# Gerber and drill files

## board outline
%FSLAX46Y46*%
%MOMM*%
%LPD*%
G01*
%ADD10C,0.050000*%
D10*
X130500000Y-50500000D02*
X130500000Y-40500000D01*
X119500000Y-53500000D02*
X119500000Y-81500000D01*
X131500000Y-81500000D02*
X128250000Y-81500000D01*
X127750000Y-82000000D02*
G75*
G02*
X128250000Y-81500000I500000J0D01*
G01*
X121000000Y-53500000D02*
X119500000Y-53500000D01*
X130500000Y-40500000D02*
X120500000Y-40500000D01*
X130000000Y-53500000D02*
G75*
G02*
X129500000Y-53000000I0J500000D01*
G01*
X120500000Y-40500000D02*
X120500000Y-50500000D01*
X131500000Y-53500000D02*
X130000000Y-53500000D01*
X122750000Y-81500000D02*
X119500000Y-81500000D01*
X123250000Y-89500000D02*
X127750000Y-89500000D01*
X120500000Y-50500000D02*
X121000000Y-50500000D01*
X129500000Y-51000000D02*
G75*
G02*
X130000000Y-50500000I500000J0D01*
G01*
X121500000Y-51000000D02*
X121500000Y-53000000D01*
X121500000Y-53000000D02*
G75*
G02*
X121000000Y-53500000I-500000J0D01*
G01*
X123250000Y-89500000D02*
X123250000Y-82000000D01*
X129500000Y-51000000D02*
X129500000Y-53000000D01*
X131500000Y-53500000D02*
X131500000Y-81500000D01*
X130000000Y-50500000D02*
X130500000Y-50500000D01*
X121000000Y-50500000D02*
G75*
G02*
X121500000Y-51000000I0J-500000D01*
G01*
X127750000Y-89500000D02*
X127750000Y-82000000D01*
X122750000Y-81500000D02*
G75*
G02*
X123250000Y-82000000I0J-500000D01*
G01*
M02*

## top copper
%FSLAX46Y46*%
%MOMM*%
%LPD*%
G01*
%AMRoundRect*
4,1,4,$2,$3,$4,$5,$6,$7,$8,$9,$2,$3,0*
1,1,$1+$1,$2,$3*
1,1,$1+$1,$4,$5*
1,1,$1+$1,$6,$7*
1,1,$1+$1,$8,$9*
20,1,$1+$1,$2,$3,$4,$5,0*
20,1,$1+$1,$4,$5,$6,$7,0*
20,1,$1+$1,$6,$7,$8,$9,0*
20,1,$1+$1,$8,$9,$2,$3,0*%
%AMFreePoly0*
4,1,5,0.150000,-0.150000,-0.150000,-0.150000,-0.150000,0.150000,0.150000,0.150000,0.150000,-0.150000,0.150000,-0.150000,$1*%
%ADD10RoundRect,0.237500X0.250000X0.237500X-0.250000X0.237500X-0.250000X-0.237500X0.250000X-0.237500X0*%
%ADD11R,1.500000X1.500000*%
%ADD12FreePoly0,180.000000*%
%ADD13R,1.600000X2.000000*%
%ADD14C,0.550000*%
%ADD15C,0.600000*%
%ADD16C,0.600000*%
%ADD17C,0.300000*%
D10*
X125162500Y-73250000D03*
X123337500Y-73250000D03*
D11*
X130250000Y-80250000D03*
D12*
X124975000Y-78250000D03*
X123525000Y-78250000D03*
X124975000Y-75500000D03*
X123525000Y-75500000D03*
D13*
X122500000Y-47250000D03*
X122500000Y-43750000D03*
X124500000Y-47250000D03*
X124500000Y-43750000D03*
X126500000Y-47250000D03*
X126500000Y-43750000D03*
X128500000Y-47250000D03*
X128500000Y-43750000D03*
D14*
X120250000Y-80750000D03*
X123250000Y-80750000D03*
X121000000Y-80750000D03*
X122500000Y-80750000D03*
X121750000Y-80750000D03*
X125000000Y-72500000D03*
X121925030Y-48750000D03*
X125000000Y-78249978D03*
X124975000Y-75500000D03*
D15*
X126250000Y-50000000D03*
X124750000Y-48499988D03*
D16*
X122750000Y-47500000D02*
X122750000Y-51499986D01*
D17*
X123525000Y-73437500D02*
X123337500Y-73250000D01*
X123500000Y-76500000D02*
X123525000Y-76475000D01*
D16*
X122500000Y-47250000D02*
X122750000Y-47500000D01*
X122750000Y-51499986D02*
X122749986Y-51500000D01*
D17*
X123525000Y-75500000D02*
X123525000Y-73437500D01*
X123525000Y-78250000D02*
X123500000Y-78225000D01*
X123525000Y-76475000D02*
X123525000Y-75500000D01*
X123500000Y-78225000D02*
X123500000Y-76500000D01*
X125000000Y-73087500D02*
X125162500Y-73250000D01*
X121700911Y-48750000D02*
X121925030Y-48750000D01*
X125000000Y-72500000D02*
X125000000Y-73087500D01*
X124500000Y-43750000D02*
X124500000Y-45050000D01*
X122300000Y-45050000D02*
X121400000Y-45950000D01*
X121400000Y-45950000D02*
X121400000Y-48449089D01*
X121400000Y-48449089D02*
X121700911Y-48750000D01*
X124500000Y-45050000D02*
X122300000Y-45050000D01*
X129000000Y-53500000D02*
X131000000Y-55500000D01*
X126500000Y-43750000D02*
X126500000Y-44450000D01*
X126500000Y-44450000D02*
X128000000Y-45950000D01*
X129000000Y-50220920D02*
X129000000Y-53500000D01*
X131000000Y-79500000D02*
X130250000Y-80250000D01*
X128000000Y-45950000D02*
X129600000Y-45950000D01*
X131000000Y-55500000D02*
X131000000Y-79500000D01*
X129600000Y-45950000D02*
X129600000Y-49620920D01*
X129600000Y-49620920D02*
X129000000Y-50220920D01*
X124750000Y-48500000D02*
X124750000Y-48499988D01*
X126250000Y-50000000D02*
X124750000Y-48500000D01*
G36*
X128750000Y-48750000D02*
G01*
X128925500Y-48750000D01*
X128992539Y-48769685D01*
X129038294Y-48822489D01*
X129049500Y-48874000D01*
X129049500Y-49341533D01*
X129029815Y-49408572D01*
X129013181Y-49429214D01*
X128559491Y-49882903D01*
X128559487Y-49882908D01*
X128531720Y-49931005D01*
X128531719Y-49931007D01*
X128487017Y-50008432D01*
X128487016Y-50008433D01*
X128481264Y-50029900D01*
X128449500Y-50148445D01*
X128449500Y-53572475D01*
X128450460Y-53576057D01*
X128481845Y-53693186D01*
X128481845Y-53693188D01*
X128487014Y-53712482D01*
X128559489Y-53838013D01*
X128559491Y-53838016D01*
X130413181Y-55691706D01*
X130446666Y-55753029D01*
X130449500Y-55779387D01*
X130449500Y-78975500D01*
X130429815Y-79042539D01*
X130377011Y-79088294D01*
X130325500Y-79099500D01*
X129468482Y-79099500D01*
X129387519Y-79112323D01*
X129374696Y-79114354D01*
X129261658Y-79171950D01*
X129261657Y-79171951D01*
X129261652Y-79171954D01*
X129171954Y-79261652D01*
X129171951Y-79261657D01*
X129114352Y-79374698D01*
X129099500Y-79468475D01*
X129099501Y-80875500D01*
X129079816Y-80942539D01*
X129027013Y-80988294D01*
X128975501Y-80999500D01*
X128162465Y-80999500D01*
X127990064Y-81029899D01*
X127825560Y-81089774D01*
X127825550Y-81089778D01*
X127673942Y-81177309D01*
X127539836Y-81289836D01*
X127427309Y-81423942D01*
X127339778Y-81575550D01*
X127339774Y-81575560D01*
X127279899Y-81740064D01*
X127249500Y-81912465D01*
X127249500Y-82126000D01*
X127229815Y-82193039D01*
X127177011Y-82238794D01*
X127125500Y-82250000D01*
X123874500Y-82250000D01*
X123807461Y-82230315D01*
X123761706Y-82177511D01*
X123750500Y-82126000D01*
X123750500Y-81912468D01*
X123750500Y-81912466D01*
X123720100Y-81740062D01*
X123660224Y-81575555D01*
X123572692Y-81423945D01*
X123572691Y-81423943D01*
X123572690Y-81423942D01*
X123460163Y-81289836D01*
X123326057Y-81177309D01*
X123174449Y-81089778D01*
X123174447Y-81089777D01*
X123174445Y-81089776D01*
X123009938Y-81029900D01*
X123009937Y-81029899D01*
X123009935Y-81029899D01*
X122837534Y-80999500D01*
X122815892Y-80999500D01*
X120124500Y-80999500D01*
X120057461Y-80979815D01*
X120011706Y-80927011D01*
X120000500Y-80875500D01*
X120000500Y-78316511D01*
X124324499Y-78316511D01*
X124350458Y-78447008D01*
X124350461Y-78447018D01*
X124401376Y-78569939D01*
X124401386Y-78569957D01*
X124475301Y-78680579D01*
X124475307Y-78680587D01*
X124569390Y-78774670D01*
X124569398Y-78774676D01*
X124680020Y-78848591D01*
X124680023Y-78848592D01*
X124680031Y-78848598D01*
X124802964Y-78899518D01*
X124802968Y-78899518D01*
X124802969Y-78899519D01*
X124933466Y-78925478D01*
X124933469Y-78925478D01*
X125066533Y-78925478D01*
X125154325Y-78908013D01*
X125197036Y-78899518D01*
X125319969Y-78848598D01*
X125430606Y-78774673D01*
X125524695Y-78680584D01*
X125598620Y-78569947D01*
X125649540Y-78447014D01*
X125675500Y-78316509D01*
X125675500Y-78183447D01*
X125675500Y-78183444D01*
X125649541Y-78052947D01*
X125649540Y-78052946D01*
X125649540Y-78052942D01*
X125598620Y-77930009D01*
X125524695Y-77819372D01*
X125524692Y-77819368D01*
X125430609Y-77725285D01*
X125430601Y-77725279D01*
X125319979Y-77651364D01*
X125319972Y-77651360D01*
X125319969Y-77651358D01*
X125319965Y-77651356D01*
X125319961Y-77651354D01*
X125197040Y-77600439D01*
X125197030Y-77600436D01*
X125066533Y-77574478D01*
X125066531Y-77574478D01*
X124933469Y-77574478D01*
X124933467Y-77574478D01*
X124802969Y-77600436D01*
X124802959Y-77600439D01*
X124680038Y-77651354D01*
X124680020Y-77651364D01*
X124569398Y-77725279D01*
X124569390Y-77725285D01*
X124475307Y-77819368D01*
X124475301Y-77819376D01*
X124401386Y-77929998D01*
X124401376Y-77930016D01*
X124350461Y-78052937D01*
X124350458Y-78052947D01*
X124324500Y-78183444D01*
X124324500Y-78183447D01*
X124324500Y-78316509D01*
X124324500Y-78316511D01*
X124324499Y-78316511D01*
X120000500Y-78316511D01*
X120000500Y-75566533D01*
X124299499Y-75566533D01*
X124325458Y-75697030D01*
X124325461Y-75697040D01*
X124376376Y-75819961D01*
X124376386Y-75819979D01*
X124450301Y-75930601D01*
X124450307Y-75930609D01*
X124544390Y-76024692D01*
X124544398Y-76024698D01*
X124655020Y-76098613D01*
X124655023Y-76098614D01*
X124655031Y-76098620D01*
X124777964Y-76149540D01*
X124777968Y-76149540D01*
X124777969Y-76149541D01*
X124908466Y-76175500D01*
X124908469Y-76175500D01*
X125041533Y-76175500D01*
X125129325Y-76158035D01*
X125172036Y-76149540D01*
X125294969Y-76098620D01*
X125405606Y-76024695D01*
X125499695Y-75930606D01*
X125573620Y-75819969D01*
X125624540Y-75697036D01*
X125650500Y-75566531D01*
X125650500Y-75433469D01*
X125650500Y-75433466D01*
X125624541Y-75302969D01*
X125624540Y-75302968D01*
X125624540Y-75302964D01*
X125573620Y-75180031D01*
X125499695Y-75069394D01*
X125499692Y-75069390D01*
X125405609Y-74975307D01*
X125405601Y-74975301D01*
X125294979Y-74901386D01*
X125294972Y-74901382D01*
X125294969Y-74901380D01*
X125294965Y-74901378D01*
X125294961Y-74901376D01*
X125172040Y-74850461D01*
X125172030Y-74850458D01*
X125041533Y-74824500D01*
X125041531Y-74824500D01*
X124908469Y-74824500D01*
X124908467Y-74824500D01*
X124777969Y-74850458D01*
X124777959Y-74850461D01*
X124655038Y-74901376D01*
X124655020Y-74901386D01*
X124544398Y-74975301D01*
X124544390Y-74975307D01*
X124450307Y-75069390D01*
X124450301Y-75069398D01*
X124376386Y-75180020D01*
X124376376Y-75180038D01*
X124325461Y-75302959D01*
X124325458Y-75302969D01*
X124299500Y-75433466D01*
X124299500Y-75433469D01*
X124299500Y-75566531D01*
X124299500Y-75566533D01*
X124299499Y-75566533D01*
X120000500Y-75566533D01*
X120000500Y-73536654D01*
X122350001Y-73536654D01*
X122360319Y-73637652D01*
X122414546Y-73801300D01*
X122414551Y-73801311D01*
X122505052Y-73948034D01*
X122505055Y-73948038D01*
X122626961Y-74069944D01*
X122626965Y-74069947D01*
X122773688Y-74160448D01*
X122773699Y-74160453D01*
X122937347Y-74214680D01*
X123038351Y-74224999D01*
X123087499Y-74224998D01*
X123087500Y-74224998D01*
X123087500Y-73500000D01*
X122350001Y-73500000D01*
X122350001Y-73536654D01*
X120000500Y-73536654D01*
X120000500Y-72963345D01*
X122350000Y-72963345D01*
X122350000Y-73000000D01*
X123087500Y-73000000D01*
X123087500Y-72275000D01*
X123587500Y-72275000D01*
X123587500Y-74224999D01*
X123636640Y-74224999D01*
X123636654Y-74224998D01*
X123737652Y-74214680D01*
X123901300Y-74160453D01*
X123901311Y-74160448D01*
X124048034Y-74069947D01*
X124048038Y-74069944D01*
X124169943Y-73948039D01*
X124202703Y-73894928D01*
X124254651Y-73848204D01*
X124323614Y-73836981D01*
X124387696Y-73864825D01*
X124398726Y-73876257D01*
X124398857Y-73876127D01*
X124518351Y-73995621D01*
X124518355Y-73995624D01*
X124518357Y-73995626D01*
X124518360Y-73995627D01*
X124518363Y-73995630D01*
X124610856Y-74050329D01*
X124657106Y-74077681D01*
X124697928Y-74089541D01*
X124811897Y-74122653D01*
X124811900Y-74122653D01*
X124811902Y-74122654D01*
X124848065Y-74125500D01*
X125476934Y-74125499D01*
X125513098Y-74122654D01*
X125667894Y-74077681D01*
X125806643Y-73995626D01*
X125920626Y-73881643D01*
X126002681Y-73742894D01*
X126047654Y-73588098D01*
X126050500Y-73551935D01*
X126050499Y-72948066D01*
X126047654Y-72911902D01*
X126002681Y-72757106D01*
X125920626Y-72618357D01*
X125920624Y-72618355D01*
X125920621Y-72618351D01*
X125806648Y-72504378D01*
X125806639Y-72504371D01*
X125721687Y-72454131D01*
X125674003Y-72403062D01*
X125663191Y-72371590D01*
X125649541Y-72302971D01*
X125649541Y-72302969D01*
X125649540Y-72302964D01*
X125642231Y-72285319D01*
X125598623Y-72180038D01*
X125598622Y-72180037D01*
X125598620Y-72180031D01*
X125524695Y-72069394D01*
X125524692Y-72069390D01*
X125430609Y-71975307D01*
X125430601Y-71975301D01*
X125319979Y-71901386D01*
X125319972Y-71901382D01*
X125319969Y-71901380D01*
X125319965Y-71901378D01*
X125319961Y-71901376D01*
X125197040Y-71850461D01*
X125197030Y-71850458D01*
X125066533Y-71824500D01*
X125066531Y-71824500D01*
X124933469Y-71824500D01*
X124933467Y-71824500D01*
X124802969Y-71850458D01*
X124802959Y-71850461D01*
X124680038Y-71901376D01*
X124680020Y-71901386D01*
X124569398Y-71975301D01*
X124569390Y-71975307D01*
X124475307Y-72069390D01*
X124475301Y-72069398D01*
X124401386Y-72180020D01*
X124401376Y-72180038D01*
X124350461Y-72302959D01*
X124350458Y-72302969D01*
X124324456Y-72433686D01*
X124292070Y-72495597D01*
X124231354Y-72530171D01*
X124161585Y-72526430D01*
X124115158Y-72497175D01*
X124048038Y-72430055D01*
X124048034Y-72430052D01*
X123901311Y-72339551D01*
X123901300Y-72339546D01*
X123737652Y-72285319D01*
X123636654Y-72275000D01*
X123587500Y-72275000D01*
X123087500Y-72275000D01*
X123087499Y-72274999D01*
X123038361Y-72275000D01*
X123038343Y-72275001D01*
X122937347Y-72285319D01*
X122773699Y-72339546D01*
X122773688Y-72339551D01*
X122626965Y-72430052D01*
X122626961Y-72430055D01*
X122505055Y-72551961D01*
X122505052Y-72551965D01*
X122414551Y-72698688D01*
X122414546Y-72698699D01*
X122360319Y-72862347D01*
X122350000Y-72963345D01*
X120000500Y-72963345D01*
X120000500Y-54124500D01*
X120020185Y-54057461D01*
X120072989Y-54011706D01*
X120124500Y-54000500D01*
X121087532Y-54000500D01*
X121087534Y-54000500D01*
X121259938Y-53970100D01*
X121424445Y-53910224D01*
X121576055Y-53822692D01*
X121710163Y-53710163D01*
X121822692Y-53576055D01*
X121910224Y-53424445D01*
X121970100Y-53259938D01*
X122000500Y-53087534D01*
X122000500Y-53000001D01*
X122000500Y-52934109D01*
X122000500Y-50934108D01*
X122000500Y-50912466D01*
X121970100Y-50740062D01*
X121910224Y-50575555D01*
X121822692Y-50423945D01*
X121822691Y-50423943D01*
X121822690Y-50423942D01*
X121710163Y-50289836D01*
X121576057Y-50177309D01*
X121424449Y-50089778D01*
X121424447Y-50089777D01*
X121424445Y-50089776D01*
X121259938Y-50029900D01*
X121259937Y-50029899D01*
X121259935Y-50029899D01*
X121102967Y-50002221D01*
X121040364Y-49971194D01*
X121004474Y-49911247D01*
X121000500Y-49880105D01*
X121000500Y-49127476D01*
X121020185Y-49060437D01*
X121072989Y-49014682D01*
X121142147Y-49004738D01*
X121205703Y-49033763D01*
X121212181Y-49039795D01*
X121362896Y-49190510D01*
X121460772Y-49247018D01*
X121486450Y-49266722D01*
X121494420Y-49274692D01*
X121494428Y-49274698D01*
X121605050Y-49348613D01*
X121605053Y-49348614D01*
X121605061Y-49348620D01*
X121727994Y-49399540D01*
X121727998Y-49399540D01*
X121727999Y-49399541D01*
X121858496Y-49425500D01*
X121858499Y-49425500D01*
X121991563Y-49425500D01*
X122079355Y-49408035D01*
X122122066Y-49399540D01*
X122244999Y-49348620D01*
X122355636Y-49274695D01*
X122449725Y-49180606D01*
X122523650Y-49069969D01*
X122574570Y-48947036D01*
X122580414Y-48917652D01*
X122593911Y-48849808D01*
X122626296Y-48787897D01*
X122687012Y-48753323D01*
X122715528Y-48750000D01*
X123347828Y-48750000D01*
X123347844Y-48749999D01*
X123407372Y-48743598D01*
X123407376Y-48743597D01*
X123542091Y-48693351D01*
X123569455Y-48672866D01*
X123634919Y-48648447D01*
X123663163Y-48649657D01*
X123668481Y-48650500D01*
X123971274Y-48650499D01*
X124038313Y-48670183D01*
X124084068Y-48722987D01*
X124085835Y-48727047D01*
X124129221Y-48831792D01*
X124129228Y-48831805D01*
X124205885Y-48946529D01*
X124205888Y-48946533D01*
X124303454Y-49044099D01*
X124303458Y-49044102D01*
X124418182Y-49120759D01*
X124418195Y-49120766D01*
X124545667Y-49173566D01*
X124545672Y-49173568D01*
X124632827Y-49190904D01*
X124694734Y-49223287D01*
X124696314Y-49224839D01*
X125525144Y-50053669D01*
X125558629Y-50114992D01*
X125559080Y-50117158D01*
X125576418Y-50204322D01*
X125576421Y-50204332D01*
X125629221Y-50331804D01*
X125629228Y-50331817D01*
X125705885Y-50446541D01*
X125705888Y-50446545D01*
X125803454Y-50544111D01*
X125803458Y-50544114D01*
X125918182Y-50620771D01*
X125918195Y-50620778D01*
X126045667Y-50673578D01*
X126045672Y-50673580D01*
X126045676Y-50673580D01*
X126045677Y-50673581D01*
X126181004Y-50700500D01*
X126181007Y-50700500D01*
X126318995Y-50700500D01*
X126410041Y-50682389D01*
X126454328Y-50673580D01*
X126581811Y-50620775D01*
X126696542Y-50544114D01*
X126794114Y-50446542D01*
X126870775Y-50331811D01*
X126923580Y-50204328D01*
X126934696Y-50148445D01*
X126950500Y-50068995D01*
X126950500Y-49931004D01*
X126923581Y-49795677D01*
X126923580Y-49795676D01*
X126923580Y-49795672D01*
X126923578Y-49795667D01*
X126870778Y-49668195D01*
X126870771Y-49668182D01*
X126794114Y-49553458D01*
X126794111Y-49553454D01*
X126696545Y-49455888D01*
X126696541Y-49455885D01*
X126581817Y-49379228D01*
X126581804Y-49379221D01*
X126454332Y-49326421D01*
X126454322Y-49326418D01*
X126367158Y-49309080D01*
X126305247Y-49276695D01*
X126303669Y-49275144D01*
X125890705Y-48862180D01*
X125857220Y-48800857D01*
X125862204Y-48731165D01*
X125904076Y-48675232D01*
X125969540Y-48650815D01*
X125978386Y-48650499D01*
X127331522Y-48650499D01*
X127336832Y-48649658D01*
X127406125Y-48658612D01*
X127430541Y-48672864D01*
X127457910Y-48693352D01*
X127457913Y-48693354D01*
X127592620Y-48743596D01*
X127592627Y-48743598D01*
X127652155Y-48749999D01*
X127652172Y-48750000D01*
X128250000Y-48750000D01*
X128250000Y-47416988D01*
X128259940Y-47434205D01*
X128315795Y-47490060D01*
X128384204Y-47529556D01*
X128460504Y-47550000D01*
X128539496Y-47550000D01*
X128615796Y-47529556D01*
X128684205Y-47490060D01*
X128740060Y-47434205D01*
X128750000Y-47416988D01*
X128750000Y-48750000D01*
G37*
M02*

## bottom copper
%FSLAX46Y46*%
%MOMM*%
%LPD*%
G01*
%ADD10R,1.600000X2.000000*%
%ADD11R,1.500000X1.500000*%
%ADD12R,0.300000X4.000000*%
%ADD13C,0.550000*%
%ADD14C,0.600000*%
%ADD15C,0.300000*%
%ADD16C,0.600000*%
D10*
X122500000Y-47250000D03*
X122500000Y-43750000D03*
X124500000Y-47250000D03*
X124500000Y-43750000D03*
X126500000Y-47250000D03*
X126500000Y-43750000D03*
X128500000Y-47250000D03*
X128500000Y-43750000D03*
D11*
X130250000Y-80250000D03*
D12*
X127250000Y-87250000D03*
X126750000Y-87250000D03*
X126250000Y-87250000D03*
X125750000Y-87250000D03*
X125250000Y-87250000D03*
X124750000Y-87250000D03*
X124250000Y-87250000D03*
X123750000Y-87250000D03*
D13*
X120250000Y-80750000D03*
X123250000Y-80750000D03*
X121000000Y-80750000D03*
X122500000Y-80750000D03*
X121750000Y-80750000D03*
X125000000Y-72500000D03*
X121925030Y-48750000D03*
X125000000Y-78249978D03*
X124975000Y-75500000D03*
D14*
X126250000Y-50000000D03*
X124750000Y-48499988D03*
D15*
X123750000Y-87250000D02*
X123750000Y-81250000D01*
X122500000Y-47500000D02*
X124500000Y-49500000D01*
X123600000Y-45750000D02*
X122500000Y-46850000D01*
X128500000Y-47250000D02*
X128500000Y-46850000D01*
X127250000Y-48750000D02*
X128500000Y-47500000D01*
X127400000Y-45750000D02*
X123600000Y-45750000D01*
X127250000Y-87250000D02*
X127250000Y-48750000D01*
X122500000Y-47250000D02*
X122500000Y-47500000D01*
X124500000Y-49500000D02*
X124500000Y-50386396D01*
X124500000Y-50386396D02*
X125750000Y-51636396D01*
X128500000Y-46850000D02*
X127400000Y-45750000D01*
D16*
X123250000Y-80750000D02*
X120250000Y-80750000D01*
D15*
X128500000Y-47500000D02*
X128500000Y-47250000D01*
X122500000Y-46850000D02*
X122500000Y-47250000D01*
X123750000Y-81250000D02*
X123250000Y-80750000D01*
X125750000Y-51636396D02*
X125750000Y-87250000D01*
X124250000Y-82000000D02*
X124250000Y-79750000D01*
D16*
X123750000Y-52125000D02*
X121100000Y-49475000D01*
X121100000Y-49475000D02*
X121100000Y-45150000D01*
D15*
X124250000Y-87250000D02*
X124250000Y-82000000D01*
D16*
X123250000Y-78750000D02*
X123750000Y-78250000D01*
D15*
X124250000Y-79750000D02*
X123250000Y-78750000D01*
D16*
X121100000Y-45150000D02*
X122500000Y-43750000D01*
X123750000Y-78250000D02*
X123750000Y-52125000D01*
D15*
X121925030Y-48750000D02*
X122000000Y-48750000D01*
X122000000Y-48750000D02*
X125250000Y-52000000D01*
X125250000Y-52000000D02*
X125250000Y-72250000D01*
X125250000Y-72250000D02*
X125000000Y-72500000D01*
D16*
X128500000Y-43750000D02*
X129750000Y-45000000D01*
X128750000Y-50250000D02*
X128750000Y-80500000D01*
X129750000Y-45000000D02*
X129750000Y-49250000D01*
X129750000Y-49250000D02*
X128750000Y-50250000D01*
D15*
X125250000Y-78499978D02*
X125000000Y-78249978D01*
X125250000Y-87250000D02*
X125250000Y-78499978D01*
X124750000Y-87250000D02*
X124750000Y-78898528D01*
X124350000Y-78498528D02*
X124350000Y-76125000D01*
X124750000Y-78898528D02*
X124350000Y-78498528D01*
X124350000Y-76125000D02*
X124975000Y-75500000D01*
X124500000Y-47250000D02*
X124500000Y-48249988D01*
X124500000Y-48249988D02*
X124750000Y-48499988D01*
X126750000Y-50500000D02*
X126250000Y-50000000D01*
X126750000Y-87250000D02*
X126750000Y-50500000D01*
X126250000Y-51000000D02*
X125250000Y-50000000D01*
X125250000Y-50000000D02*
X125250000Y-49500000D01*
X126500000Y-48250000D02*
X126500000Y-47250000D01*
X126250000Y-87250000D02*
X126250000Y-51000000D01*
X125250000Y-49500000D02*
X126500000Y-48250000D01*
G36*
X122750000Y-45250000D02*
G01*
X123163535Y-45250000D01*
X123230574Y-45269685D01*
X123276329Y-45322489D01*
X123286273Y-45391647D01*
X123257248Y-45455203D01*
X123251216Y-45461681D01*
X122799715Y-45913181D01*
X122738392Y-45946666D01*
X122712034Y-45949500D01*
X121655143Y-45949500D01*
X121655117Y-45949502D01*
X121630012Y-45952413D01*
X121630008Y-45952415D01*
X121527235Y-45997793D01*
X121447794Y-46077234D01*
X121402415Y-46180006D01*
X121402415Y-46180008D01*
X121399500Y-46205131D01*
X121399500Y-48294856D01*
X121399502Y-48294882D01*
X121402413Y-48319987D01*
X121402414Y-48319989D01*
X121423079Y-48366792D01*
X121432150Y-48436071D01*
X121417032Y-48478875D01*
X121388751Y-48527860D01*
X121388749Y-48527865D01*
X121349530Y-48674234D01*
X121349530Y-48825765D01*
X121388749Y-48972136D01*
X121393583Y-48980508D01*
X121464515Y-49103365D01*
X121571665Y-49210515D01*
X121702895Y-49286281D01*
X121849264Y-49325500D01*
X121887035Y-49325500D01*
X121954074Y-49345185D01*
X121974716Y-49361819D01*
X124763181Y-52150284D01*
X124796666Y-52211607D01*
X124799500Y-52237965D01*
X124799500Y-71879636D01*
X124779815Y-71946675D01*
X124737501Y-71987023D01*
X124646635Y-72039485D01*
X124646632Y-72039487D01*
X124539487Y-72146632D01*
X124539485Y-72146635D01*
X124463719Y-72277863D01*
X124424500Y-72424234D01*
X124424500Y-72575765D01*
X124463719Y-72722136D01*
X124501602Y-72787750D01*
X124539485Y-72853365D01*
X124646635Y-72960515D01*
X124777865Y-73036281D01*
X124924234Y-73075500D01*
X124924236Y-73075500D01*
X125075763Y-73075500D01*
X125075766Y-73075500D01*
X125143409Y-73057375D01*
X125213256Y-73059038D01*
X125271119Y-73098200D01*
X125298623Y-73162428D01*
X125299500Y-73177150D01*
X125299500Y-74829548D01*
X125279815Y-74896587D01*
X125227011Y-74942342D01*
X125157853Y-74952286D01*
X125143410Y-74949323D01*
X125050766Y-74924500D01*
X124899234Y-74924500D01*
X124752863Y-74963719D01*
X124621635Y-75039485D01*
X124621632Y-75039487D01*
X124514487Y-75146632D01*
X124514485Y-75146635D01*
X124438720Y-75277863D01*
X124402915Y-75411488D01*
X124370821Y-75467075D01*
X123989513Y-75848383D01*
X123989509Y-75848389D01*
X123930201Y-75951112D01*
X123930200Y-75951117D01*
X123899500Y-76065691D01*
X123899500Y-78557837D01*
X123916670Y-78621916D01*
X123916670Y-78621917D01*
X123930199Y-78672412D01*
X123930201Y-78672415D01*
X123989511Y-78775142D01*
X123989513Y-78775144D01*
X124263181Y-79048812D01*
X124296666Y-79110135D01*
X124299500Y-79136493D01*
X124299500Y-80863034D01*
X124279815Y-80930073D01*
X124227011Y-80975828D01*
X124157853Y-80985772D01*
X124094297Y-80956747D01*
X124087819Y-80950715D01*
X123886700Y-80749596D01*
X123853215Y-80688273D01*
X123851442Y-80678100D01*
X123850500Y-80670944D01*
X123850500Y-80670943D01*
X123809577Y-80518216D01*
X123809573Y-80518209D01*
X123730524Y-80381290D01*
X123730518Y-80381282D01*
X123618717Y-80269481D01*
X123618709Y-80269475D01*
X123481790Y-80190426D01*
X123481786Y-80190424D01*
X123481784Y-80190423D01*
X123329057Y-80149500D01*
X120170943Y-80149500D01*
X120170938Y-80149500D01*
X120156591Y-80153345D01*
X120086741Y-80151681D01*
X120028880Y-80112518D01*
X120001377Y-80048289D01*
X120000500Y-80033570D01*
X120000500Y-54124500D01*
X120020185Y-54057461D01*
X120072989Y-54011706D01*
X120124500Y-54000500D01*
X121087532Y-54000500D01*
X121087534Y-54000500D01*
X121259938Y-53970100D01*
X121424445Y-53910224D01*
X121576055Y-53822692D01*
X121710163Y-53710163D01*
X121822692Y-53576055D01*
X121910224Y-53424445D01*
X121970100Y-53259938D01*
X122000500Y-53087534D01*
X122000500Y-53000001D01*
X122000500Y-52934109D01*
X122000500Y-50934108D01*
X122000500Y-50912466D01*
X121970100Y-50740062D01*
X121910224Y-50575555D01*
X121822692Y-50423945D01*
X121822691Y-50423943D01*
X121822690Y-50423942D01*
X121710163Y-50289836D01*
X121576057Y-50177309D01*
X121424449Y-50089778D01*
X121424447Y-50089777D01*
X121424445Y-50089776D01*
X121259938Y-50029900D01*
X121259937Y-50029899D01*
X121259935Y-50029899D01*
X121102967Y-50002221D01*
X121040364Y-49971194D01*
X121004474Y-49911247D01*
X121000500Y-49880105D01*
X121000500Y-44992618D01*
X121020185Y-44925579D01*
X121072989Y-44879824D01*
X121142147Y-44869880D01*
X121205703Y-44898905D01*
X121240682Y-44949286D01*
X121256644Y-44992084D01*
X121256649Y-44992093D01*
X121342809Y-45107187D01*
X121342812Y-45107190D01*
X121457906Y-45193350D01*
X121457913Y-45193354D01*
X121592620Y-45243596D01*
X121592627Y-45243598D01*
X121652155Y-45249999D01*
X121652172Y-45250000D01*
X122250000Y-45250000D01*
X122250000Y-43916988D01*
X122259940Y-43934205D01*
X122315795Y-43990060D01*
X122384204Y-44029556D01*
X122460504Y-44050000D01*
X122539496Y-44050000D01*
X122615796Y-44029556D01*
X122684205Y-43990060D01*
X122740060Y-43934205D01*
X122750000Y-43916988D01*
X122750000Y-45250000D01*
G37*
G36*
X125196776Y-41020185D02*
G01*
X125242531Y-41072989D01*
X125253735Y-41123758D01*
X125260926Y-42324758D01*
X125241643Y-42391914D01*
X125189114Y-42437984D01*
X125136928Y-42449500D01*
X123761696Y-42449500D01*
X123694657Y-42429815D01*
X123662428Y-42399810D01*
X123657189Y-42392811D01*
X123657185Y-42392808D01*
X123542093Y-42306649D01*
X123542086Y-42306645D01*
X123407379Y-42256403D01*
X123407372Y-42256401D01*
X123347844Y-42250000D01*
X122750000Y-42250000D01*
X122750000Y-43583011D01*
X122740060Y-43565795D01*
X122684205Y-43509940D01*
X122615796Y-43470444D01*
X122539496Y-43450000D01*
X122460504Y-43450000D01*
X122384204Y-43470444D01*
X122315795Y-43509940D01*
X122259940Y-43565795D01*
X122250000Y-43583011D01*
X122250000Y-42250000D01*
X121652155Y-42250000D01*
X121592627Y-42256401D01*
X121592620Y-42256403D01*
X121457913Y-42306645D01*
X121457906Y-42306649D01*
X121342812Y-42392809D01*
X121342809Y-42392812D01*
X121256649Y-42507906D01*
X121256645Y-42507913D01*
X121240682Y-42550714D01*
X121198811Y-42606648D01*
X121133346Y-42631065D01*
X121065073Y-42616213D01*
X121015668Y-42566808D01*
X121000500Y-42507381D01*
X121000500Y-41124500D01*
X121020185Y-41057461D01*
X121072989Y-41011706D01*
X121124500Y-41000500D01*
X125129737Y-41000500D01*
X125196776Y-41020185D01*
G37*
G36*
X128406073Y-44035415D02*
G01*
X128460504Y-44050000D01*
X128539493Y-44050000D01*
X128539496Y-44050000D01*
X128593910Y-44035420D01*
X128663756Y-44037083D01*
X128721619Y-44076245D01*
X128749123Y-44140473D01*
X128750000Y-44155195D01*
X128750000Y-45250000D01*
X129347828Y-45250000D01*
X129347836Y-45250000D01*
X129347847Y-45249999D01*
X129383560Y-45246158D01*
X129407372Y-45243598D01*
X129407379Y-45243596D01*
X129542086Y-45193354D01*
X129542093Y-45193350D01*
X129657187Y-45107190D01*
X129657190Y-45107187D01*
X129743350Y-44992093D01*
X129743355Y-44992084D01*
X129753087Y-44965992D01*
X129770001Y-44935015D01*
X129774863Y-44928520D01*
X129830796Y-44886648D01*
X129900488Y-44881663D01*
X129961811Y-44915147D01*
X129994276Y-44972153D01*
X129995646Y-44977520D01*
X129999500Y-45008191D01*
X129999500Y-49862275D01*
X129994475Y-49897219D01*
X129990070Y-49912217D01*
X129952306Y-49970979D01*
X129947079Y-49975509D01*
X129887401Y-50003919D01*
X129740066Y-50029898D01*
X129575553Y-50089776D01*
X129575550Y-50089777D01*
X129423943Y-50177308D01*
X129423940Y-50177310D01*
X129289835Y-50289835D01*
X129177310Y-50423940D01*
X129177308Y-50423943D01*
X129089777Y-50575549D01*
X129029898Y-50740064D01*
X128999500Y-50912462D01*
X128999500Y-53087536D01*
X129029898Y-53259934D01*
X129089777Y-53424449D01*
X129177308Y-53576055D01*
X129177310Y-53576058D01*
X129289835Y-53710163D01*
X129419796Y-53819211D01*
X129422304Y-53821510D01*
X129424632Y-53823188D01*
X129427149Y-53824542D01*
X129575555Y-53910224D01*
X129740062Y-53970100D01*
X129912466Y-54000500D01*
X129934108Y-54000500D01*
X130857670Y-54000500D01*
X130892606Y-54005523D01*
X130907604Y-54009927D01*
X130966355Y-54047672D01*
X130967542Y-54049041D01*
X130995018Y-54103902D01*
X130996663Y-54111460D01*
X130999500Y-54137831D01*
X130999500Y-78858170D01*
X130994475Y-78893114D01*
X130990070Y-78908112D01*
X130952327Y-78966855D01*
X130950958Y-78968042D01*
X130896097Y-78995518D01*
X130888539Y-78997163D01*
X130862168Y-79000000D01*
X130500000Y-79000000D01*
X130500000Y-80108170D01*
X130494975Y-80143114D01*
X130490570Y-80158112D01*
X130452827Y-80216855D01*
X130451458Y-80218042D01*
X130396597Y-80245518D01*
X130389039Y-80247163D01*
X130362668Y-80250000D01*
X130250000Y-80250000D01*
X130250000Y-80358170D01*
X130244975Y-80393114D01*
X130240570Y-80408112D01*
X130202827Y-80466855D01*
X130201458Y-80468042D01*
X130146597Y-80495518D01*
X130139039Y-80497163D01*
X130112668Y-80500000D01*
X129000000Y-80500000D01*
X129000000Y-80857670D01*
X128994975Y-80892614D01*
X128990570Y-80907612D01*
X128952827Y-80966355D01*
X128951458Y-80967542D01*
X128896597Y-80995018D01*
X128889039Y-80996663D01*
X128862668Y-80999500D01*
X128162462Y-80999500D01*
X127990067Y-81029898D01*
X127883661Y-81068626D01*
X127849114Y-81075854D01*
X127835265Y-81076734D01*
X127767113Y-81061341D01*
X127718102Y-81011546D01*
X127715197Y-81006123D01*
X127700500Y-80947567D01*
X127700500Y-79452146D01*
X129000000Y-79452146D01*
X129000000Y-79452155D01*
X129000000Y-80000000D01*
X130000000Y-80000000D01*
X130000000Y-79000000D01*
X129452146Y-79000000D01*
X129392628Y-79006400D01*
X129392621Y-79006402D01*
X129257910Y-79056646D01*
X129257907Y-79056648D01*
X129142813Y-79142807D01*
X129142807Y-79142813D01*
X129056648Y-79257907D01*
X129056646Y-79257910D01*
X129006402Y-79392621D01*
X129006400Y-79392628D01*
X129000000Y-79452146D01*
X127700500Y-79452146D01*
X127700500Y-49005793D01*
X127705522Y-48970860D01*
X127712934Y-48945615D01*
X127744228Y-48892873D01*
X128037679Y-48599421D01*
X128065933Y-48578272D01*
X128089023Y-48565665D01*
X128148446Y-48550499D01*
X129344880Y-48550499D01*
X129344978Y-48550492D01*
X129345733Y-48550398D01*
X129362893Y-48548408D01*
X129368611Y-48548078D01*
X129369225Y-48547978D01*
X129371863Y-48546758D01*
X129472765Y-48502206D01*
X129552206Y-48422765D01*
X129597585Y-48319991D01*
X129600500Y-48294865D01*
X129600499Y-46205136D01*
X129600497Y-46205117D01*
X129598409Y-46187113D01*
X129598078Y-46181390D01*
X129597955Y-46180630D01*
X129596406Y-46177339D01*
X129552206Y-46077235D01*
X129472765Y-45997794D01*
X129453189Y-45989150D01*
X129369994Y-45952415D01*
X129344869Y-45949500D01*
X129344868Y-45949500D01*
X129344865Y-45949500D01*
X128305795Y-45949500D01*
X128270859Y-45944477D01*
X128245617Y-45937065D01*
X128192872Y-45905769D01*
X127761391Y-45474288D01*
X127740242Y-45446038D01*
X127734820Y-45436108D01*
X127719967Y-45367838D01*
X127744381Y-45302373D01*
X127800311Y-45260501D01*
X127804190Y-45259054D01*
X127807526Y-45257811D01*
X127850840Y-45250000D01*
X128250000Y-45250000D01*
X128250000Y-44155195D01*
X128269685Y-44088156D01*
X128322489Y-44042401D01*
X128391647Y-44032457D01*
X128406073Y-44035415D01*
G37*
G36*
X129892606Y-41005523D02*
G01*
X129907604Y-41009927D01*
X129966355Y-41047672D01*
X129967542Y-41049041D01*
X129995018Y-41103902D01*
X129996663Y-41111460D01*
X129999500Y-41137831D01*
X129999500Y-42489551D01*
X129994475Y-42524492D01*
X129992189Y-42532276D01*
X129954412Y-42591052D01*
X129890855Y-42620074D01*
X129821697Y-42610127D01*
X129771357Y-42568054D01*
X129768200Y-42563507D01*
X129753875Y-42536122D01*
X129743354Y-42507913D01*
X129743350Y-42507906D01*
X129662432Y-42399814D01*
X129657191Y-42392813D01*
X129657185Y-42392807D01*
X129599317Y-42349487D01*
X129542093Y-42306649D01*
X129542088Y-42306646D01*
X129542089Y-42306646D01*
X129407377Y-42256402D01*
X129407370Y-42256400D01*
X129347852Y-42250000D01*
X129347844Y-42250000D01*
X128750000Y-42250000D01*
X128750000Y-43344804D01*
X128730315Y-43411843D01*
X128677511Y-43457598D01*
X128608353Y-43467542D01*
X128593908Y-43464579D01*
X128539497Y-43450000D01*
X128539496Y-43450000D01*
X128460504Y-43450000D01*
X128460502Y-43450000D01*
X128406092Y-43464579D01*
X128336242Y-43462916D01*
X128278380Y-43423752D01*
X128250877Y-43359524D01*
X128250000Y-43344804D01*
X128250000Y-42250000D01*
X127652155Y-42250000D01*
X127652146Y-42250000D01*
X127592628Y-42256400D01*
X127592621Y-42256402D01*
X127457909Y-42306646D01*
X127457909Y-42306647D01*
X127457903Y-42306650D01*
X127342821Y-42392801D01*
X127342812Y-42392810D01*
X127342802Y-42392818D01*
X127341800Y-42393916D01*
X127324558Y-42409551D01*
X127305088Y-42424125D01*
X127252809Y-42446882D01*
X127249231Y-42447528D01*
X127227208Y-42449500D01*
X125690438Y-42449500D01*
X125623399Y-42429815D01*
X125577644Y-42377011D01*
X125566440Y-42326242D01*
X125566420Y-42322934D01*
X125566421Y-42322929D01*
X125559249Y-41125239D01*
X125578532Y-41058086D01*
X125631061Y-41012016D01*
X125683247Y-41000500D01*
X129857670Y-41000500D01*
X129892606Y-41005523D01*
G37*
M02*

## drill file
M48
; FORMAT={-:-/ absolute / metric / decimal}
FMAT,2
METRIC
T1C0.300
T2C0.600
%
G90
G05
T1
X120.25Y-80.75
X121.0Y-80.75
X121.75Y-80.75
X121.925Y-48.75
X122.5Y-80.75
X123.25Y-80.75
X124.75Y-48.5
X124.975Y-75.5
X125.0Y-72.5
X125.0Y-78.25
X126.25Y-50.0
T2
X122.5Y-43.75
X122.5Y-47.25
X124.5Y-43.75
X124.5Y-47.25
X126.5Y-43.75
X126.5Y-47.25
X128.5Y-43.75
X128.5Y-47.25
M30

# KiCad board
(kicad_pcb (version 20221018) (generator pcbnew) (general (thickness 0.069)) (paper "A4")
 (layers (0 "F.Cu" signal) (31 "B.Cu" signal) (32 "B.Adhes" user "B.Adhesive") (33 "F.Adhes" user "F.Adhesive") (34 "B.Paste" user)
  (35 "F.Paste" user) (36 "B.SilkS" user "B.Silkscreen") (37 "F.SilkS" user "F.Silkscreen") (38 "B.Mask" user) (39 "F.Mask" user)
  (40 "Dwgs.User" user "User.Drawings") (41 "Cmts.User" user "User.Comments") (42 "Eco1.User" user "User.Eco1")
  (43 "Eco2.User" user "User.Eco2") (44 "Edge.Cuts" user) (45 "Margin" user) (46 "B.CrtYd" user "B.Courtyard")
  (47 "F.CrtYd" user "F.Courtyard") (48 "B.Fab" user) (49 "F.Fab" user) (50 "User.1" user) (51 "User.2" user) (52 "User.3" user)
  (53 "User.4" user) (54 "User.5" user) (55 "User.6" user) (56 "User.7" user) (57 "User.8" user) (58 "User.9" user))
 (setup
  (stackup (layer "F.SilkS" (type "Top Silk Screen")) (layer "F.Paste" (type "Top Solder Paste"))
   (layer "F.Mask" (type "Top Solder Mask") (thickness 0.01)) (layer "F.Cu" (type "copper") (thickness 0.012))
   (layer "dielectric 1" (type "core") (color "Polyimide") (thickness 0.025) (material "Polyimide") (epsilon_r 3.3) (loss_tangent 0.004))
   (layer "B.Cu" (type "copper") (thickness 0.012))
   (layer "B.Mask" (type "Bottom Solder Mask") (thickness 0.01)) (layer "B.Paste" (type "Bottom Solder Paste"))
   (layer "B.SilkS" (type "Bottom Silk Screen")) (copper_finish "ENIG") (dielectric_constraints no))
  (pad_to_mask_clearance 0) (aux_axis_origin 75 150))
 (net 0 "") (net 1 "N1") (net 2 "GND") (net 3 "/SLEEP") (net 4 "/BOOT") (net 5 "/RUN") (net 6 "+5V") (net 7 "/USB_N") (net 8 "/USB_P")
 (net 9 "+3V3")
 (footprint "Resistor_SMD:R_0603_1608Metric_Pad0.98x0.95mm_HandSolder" (layer "F.Cu") (at 124.25 73.25 180)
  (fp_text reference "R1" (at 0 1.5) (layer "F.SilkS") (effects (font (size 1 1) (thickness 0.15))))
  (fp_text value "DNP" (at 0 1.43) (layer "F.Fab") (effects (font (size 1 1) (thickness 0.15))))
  (pad "1" smd roundrect (at -0.9125 0 180) (size 0.975 0.95) (layers "F.Cu" "F.Paste" "F.Mask") (roundrect_rratio 0.25) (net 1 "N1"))
  (pad "2" smd roundrect (at 0.9125 0 180) (size 0.975 0.95) (layers "F.Cu" "F.Paste" "F.Mask") (roundrect_rratio 0.25) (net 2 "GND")))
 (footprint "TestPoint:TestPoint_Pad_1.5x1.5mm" (layer "F.Cu") (at 130.25 80.25)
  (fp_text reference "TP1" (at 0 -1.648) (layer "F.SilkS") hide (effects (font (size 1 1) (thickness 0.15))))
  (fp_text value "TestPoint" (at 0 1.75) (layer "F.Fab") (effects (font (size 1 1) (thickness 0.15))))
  (pad "1" smd rect (at 0 0) (size 1.5 1.5) (layers "F.Cu" "F.Mask") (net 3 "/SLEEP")))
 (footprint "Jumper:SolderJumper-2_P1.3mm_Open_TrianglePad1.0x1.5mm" (layer "F.Cu") (at 124.25 78.25 180) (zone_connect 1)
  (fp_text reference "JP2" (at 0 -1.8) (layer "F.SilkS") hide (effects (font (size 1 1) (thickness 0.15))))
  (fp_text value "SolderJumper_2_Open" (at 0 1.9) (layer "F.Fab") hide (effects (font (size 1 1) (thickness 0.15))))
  (pad "1" smd custom (at -0.725 0 180) (size 0.3 0.3) (layers "F.Cu" "F.Mask") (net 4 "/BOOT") (zone_connect 2) (thermal_bridge_angle 45)
   (options (clearance outline) (anchor rect)) (primitives))
  (pad "2" smd custom (at 0.725 0 180) (size 0.3 0.3) (layers "F.Cu" "F.Mask") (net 2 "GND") (zone_connect 2) (thermal_bridge_angle 45)
   (options (clearance outline) (anchor rect)) (primitives)))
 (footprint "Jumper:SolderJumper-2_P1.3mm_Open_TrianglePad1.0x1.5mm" (layer "F.Cu") (at 124.25 75.5 180) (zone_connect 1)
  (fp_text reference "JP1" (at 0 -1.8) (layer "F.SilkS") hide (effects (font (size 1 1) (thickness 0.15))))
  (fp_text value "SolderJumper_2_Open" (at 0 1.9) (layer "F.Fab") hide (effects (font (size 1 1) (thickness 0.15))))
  (pad "1" smd custom (at -0.725 0 180) (size 0.3 0.3) (layers "F.Cu" "F.Mask") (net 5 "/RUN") (zone_connect 2) (thermal_bridge_angle 45)
   (options (clearance outline) (anchor rect)) (primitives))
  (pad "2" smd custom (at 0.725 0 180) (size 0.3 0.3) (layers "F.Cu" "F.Mask") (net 2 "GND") (zone_connect 2) (thermal_bridge_angle 45)
   (options (clearance outline) (anchor rect)) (primitives)))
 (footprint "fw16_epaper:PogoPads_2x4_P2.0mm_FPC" (layer "B.Cu") (at 125.5 45.5 180)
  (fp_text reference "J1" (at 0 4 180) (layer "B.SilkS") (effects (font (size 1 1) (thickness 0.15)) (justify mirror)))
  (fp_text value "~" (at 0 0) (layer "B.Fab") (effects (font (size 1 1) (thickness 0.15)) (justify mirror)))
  (pad "1" thru_hole rect (at 3 -1.75 180) (size 1.6 2) (drill 0.6) (layers "*.Cu" "B.Mask") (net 2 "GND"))
  (pad "2" thru_hole rect (at 3 1.75 180) (size 1.6 2) (drill 0.6) (layers "*.Cu" "B.Mask") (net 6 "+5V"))
  (pad "3" thru_hole rect (at 1 -1.75 180) (size 1.6 2) (drill 0.6) (layers "*.Cu" "B.Mask") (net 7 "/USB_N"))
  (pad "4" thru_hole rect (at 1 1.75 180) (size 1.6 2) (drill 0.6) (layers "*.Cu" "B.Mask") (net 1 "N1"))
  (pad "5" thru_hole rect (at -1 -1.75 180) (size 1.6 2) (drill 0.6) (layers "*.Cu" "B.Mask") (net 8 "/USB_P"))
  (pad "6" thru_hole rect (at -1 1.75 180) (size 1.6 2) (drill 0.6) (layers "*.Cu" "B.Mask") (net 3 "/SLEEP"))
  (pad "7" thru_hole rect (at -3 -1.75 180) (size 1.6 2) (drill 0.6) (layers "*.Cu" "B.Mask") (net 2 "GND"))
  (pad "8" thru_hole rect (at -3 1.75 180) (size 1.6 2) (drill 0.6) (layers "*.Cu" "B.Mask") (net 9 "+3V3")))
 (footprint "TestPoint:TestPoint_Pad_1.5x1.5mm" (layer "B.Cu") (at 130.25 80.25 180)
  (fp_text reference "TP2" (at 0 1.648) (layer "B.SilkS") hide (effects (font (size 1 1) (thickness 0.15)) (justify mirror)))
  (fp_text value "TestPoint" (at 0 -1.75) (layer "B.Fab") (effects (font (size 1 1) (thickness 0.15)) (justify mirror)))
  (pad "1" smd rect (at 0 0 180) (size 1.5 1.5) (layers "B.Cu" "B.Mask") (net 9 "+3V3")))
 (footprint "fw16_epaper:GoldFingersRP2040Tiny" (layer "B.Cu") (at 125.5 87.25 180)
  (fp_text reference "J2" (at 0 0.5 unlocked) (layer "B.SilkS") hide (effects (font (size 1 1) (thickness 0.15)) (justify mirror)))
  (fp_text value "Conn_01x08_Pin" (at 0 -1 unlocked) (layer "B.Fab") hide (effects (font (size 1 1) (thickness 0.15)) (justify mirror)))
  (pad "1" smd rect (at -1.75 0) (size 0.3 4) (layers "B.Cu" "B.Paste" "B.Mask") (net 2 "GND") (thermal_bridge_angle 45))
  (pad "2" smd rect (at -1.25 0) (size 0.3 4) (layers "B.Cu" "B.Paste" "B.Mask") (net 7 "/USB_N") (thermal_bridge_angle 45))
  (pad "3" smd rect (at -0.75 0) (size 0.3 4) (layers "B.Cu" "B.Paste" "B.Mask") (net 8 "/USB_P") (thermal_bridge_angle 45))
  (pad "4" smd rect (at -0.25 0) (size 0.3 4) (layers "B.Cu" "B.Paste" "B.Mask") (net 2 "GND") (thermal_bridge_angle 45))
  (pad "5" smd rect (at 0.25 0) (size 0.3 4) (layers "B.Cu" "B.Paste" "B.Mask") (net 4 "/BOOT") (thermal_bridge_angle 45))
  (pad "6" smd rect (at 0.75 0) (size 0.3 4) (layers "B.Cu" "B.Paste" "B.Mask") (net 5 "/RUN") (thermal_bridge_angle 45))
  (pad "7" smd rect (at 1.25 0) (size 0.3 4) (layers "B.Cu" "B.Paste" "B.Mask") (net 6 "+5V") (thermal_bridge_angle 45))
  (pad "8" smd rect (at 1.75 0) (size 0.3 4) (layers "B.Cu" "B.Paste" "B.Mask") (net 2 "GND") (thermal_bridge_angle 45)))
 (gr_line (start 130.5 50.5) (end 130.5 40.5) (stroke (width 0.05) (type default)) (layer "Edge.Cuts"))
 (gr_line (start 119.5 53.5) (end 119.5 81.5) (stroke (width 0.05) (type default)) (layer "Edge.Cuts"))
 (gr_line (start 131.5 81.5) (end 128.25 81.5) (stroke (width 0.05) (type default)) (layer "Edge.Cuts"))
 (gr_arc (start 127.75 82) (mid 127.896447 81.646447) (end 128.25 81.5) (stroke (width 0.05) (type default)) (layer "Edge.Cuts"))
 (gr_line (start 121 53.5) (end 119.5 53.5) (stroke (width 0.05) (type default)) (layer "Edge.Cuts"))
 (gr_line (start 130.5 40.5) (end 120.5 40.5) (stroke (width 0.05) (type default)) (layer "Edge.Cuts"))
 (gr_arc (start 130 53.5) (mid 129.646447 53.353553) (end 129.5 53) (stroke (width 0.05) (type default)) (layer "Edge.Cuts"))
 (gr_line (start 120.5 40.5) (end 120.5 50.5) (stroke (width 0.05) (type default)) (layer "Edge.Cuts"))
 (gr_line (start 131.5 53.5) (end 130 53.5) (stroke (width 0.05) (type default)) (layer "Edge.Cuts"))
 (gr_line (start 122.75 81.5) (end 119.5 81.5) (stroke (width 0.05) (type default)) (layer "Edge.Cuts"))
 (gr_line (start 123.25 89.5) (end 127.75 89.5) (stroke (width 0.05) (type default)) (layer "Edge.Cuts"))
 (gr_line (start 120.5 50.5) (end 121 50.5) (stroke (width 0.05) (type default)) (layer "Edge.Cuts"))
 (gr_arc (start 129.5 51) (mid 129.646447 50.646447) (end 130 50.5) (stroke (width 0.05) (type default)) (layer "Edge.Cuts"))
 (gr_line (start 121.5 51) (end 121.5 53) (stroke (width 0.05) (type default)) (layer "Edge.Cuts"))
 (gr_arc (start 121.5 53) (mid 121.353553 53.353553) (end 121 53.5) (stroke (width 0.05) (type default)) (layer "Edge.Cuts"))
 (gr_line (start 123.25 89.5) (end 123.25 82) (stroke (width 0.05) (type default)) (layer "Edge.Cuts"))
 (gr_line (start 129.5 51) (end 129.5 53) (stroke (width 0.05) (type default)) (layer "Edge.Cuts"))
 (gr_line (start 131.5 53.5) (end 131.5 81.5) (stroke (width 0.05) (type default)) (layer "Edge.Cuts"))
 (gr_line (start 130 50.5) (end 130.5 50.5) (stroke (width 0.05) (type default)) (layer "Edge.Cuts"))
 (gr_arc (start 121 50.5) (mid 121.353553 50.646447) (end 121.5 51) (stroke (width 0.05) (type default)) (layer "Edge.Cuts"))
 (gr_line (start 127.75 89.5) (end 127.75 82) (stroke (width 0.05) (type default)) (layer "Edge.Cuts"))
 (gr_arc (start 122.75 81.5) (mid 123.103553 81.646447) (end 123.25 82) (stroke (width 0.05) (type default)) (layer "Edge.Cuts"))
 (segment (start 122.75 47.5) (end 122.75 51.499986) (width 0.6) (layer "F.Cu") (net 2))
 (segment (start 123.525 73.4375) (end 123.3375 73.25) (width 0.3) (layer "F.Cu") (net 2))
 (segment (start 123.5 76.5) (end 123.525 76.475) (width 0.3) (layer "F.Cu") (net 2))
 (segment (start 122.5 47.25) (end 122.75 47.5) (width 0.6) (layer "F.Cu") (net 2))
 (segment (start 122.75 51.499986) (end 122.749986 51.5) (width 0.6) (layer "F.Cu") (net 2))
 (segment (start 123.525 75.5) (end 123.525 73.4375) (width 0.3) (layer "F.Cu") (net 2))
 (segment (start 123.525 78.25) (end 123.5 78.225) (width 0.3) (layer "F.Cu") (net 2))
 (segment (start 123.525 76.475) (end 123.525 75.5) (width 0.3) (layer "F.Cu") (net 2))
 (segment (start 123.5 78.225) (end 123.5 76.5) (width 0.3) (layer "F.Cu") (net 2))
 (via (at 120.25 80.75) (size 0.55) (drill 0.3) (layers "F.Cu" "B.Cu") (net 2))
 (via (at 123.25 80.75) (size 0.55) (drill 0.3) (layers "F.Cu" "B.Cu") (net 2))
 (via (at 121 80.75) (size 0.55) (drill 0.3) (layers "F.Cu" "B.Cu") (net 2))
 (via (at 122.5 80.75) (size 0.55) (drill 0.3) (layers "F.Cu" "B.Cu") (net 2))
 (via (at 121.75 80.75) (size 0.55) (drill 0.3) (layers "F.Cu" "B.Cu") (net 2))
 (segment (start 123.75 87.25) (end 123.75 81.25) (width 0.3) (layer "B.Cu") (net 2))
 (segment (start 122.5 47.5) (end 124.5 49.5) (width 0.3) (layer "B.Cu") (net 2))
 (segment (start 123.6 45.75) (end 122.5 46.85) (width 0.3) (layer "B.Cu") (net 2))
 (segment (start 128.5 47.25) (end 128.5 46.85) (width 0.3) (layer "B.Cu") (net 2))
 (segment (start 127.25 48.75) (end 128.5 47.5) (width 0.3) (layer "B.Cu") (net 2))
 (segment (start 127.4 45.75) (end 123.6 45.75) (width 0.3) (layer "B.Cu") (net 2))
 (segment (start 127.25 87.25) (end 127.25 48.75) (width 0.3) (layer "B.Cu") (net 2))
 (segment (start 122.5 47.25) (end 122.5 47.5) (width 0.3) (layer "B.Cu") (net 2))
 (segment (start 124.5 49.5) (end 124.5 50.386396) (width 0.3) (layer "B.Cu") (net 2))
 (segment (start 124.5 50.386396) (end 125.75 51.636396) (width 0.3) (layer "B.Cu") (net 2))
 (segment (start 128.5 46.85) (end 127.4 45.75) (width 0.3) (layer "B.Cu") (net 2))
 (segment (start 123.25 80.75) (end 120.25 80.75) (width 0.6) (layer "B.Cu") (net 2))
 (segment (start 128.5 47.5) (end 128.5 47.25) (width 0.3) (layer "B.Cu") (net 2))
 (segment (start 122.5 46.85) (end 122.5 47.25) (width 0.3) (layer "B.Cu") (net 2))
 (segment (start 123.75 81.25) (end 123.25 80.75) (width 0.3) (layer "B.Cu") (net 2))
 (segment (start 125.75 51.636396) (end 125.75 87.25) (width 0.3) (layer "B.Cu") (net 2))
 (segment (start 124.25 82) (end 124.25 79.75) (width 0.3) (layer "B.Cu") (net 6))
 (segment (start 123.75 52.125) (end 121.1 49.475) (width 0.6) (layer "B.Cu") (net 6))
 (segment (start 121.1 49.475) (end 121.1 45.15) (width 0.6) (layer "B.Cu") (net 6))
 (segment (start 124.25 87.25) (end 124.25 82) (width 0.3) (layer "B.Cu") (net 6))
 (segment (start 123.25 78.75) (end 123.75 78.25) (width 0.6) (layer "B.Cu") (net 6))
 (segment (start 124.25 79.75) (end 123.25 78.75) (width 0.3) (layer "B.Cu") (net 6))
 (segment (start 121.1 45.15) (end 122.5 43.75) (width 0.6) (layer "B.Cu") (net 6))
 (segment (start 123.75 78.25) (end 123.75 52.125) (width 0.6) (layer "B.Cu") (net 6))
 (segment (start 125 73.0875) (end 125.1625 73.25) (width 0.3) (layer "F.Cu") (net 1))
 (segment (start 121.700911 48.75) (end 121.92503 48.75) (width 0.3) (layer "F.Cu") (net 1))
 (segment (start 125 72.5) (end 125 73.0875) (width 0.3) (layer "F.Cu") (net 1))
 (segment (start 124.5 43.75) (end 124.5 45.05) (width 0.3) (layer "F.Cu") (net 1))
 (segment (start 122.3 45.05) (end 121.4 45.95) (width 0.3) (layer "F.Cu") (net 1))
 (segment (start 121.4 45.95) (end 121.4 48.449089) (width 0.3) (layer "F.Cu") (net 1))
 (segment (start 121.4 48.449089) (end 121.700911 48.75) (width 0.3) (layer "F.Cu") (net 1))
 (segment (start 124.5 45.05) (end 122.3 45.05) (width 0.3) (layer "F.Cu") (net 1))
 (via (at 125 72.5) (size 0.55) (drill 0.3) (layers "F.Cu" "B.Cu") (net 1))
 (via (at 121.92503 48.75) (size 0.55) (drill 0.3) (layers "F.Cu" "B.Cu") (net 1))
 (segment (start 121.92503 48.75) (end 122 48.75) (width 0.3) (layer "B.Cu") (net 1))
 (segment (start 122 48.75) (end 125.25 52) (width 0.3) (layer "B.Cu") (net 1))
 (segment (start 125.25 52) (end 125.25 72.25) (width 0.3) (layer "B.Cu") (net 1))
 (segment (start 125.25 72.25) (end 125 72.5) (width 0.3) (layer "B.Cu") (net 1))
 (segment (start 128.5 43.75) (end 129.75 45) (width 0.6) (layer "B.Cu") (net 9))
 (segment (start 128.75 50.25) (end 128.75 80.5) (width 0.6) (layer "B.Cu") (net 9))
 (segment (start 129.75 45) (end 129.75 49.25) (width 0.6) (layer "B.Cu") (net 9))
 (segment (start 129.75 49.25) (end 128.75 50.25) (width 0.6) (layer "B.Cu") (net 9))
 (segment (start 129 53.5) (end 131 55.5) (width 0.3) (layer "F.Cu") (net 3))
 (segment (start 126.5 43.75) (end 126.5 44.45) (width 0.3) (layer "F.Cu") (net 3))
 (segment (start 126.5 44.45) (end 128 45.95) (width 0.3) (layer "F.Cu") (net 3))
 (segment (start 129 50.22092) (end 129 53.5) (width 0.3) (layer "F.Cu") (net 3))
 (segment (start 131 79.5) (end 130.25 80.25) (width 0.3) (layer "F.Cu") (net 3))
 (segment (start 128 45.95) (end 129.6 45.95) (width 0.3) (layer "F.Cu") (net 3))
 (segment (start 131 55.5) (end 131 79.5) (width 0.3) (layer "F.Cu") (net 3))
 (segment (start 129.6 45.95) (end 129.6 49.62092) (width 0.3) (layer "F.Cu") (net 3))
 (segment (start 129.6 49.62092) (end 129 50.22092) (width 0.3) (layer "F.Cu") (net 3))
 (via (at 125 78.249978) (size 0.55) (drill 0.3) (layers "F.Cu" "B.Cu") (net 4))
 (segment (start 125.25 78.499978) (end 125 78.249978) (width 0.3) (layer "B.Cu") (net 4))
 (segment (start 125.25 87.25) (end 125.25 78.499978) (width 0.3) (layer "B.Cu") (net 4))
 (via (at 124.975 75.5) (size 0.55) (drill 0.3) (layers "F.Cu" "B.Cu") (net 5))
 (segment (start 124.75 87.25) (end 124.75 78.898528) (width 0.3) (layer "B.Cu") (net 5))
 (segment (start 124.35 78.498528) (end 124.35 76.125) (width 0.3) (layer "B.Cu") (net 5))
 (segment (start 124.75 78.898528) (end 124.35 78.498528) (width 0.3) (layer "B.Cu") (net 5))
 (segment (start 124.35 76.125) (end 124.975 75.5) (width 0.3) (layer "B.Cu") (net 5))
 (segment (start 124.75 48.5) (end 124.75 48.499988) (width 0.3) (layer "F.Cu") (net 7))
 (segment (start 126.25 50) (end 124.75 48.5) (width 0.3) (layer "F.Cu") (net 7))
 (via (at 126.25 50) (size 0.6) (drill 0.3) (layers "F.Cu" "B.Cu") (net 7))
 (via (at 124.75 48.499988) (size 0.6) (drill 0.3) (layers "F.Cu" "B.Cu") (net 7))
 (segment (start 124.5 47.25) (end 124.5 48.249988) (width 0.3) (layer "B.Cu") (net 7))
 (segment (start 124.5 48.249988) (end 124.75 48.499988) (width 0.3) (layer "B.Cu") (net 7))
 (segment (start 126.75 50.5) (end 126.25 50) (width 0.3) (layer "B.Cu") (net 7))
 (segment (start 126.75 87.25) (end 126.75 50.5) (width 0.3) (layer "B.Cu") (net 7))
 (segment (start 126.25 51) (end 125.25 50) (width 0.3) (layer "B.Cu") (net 8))
 (segment (start 125.25 50) (end 125.25 49.5) (width 0.3) (layer "B.Cu") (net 8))
 (segment (start 126.5 48.25) (end 126.5 47.25) (width 0.3) (layer "B.Cu") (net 8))
 (segment (start 126.25 87.25) (end 126.25 51) (width 0.3) (layer "B.Cu") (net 8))
 (segment (start 125.25 49.5) (end 126.5 48.25) (width 0.3) (layer "B.Cu") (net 8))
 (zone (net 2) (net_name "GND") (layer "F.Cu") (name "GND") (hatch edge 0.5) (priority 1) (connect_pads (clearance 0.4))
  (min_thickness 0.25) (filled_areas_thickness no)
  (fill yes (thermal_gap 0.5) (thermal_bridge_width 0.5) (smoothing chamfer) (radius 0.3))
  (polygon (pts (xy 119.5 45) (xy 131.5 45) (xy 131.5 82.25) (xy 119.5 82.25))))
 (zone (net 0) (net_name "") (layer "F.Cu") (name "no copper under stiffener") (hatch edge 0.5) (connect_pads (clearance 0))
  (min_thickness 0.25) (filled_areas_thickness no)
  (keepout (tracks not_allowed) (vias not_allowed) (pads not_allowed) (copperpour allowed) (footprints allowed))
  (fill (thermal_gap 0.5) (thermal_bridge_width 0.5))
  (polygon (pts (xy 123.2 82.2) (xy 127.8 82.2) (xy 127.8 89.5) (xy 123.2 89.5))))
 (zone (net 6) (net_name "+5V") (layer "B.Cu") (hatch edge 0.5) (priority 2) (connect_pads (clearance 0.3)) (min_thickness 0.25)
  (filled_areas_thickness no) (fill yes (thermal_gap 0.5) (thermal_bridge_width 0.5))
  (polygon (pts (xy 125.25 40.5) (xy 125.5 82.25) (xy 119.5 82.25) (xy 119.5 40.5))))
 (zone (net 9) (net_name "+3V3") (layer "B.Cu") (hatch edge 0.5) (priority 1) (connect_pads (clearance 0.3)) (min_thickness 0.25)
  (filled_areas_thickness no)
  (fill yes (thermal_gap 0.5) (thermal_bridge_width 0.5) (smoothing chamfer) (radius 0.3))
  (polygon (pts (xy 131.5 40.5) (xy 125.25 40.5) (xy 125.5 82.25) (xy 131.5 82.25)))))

